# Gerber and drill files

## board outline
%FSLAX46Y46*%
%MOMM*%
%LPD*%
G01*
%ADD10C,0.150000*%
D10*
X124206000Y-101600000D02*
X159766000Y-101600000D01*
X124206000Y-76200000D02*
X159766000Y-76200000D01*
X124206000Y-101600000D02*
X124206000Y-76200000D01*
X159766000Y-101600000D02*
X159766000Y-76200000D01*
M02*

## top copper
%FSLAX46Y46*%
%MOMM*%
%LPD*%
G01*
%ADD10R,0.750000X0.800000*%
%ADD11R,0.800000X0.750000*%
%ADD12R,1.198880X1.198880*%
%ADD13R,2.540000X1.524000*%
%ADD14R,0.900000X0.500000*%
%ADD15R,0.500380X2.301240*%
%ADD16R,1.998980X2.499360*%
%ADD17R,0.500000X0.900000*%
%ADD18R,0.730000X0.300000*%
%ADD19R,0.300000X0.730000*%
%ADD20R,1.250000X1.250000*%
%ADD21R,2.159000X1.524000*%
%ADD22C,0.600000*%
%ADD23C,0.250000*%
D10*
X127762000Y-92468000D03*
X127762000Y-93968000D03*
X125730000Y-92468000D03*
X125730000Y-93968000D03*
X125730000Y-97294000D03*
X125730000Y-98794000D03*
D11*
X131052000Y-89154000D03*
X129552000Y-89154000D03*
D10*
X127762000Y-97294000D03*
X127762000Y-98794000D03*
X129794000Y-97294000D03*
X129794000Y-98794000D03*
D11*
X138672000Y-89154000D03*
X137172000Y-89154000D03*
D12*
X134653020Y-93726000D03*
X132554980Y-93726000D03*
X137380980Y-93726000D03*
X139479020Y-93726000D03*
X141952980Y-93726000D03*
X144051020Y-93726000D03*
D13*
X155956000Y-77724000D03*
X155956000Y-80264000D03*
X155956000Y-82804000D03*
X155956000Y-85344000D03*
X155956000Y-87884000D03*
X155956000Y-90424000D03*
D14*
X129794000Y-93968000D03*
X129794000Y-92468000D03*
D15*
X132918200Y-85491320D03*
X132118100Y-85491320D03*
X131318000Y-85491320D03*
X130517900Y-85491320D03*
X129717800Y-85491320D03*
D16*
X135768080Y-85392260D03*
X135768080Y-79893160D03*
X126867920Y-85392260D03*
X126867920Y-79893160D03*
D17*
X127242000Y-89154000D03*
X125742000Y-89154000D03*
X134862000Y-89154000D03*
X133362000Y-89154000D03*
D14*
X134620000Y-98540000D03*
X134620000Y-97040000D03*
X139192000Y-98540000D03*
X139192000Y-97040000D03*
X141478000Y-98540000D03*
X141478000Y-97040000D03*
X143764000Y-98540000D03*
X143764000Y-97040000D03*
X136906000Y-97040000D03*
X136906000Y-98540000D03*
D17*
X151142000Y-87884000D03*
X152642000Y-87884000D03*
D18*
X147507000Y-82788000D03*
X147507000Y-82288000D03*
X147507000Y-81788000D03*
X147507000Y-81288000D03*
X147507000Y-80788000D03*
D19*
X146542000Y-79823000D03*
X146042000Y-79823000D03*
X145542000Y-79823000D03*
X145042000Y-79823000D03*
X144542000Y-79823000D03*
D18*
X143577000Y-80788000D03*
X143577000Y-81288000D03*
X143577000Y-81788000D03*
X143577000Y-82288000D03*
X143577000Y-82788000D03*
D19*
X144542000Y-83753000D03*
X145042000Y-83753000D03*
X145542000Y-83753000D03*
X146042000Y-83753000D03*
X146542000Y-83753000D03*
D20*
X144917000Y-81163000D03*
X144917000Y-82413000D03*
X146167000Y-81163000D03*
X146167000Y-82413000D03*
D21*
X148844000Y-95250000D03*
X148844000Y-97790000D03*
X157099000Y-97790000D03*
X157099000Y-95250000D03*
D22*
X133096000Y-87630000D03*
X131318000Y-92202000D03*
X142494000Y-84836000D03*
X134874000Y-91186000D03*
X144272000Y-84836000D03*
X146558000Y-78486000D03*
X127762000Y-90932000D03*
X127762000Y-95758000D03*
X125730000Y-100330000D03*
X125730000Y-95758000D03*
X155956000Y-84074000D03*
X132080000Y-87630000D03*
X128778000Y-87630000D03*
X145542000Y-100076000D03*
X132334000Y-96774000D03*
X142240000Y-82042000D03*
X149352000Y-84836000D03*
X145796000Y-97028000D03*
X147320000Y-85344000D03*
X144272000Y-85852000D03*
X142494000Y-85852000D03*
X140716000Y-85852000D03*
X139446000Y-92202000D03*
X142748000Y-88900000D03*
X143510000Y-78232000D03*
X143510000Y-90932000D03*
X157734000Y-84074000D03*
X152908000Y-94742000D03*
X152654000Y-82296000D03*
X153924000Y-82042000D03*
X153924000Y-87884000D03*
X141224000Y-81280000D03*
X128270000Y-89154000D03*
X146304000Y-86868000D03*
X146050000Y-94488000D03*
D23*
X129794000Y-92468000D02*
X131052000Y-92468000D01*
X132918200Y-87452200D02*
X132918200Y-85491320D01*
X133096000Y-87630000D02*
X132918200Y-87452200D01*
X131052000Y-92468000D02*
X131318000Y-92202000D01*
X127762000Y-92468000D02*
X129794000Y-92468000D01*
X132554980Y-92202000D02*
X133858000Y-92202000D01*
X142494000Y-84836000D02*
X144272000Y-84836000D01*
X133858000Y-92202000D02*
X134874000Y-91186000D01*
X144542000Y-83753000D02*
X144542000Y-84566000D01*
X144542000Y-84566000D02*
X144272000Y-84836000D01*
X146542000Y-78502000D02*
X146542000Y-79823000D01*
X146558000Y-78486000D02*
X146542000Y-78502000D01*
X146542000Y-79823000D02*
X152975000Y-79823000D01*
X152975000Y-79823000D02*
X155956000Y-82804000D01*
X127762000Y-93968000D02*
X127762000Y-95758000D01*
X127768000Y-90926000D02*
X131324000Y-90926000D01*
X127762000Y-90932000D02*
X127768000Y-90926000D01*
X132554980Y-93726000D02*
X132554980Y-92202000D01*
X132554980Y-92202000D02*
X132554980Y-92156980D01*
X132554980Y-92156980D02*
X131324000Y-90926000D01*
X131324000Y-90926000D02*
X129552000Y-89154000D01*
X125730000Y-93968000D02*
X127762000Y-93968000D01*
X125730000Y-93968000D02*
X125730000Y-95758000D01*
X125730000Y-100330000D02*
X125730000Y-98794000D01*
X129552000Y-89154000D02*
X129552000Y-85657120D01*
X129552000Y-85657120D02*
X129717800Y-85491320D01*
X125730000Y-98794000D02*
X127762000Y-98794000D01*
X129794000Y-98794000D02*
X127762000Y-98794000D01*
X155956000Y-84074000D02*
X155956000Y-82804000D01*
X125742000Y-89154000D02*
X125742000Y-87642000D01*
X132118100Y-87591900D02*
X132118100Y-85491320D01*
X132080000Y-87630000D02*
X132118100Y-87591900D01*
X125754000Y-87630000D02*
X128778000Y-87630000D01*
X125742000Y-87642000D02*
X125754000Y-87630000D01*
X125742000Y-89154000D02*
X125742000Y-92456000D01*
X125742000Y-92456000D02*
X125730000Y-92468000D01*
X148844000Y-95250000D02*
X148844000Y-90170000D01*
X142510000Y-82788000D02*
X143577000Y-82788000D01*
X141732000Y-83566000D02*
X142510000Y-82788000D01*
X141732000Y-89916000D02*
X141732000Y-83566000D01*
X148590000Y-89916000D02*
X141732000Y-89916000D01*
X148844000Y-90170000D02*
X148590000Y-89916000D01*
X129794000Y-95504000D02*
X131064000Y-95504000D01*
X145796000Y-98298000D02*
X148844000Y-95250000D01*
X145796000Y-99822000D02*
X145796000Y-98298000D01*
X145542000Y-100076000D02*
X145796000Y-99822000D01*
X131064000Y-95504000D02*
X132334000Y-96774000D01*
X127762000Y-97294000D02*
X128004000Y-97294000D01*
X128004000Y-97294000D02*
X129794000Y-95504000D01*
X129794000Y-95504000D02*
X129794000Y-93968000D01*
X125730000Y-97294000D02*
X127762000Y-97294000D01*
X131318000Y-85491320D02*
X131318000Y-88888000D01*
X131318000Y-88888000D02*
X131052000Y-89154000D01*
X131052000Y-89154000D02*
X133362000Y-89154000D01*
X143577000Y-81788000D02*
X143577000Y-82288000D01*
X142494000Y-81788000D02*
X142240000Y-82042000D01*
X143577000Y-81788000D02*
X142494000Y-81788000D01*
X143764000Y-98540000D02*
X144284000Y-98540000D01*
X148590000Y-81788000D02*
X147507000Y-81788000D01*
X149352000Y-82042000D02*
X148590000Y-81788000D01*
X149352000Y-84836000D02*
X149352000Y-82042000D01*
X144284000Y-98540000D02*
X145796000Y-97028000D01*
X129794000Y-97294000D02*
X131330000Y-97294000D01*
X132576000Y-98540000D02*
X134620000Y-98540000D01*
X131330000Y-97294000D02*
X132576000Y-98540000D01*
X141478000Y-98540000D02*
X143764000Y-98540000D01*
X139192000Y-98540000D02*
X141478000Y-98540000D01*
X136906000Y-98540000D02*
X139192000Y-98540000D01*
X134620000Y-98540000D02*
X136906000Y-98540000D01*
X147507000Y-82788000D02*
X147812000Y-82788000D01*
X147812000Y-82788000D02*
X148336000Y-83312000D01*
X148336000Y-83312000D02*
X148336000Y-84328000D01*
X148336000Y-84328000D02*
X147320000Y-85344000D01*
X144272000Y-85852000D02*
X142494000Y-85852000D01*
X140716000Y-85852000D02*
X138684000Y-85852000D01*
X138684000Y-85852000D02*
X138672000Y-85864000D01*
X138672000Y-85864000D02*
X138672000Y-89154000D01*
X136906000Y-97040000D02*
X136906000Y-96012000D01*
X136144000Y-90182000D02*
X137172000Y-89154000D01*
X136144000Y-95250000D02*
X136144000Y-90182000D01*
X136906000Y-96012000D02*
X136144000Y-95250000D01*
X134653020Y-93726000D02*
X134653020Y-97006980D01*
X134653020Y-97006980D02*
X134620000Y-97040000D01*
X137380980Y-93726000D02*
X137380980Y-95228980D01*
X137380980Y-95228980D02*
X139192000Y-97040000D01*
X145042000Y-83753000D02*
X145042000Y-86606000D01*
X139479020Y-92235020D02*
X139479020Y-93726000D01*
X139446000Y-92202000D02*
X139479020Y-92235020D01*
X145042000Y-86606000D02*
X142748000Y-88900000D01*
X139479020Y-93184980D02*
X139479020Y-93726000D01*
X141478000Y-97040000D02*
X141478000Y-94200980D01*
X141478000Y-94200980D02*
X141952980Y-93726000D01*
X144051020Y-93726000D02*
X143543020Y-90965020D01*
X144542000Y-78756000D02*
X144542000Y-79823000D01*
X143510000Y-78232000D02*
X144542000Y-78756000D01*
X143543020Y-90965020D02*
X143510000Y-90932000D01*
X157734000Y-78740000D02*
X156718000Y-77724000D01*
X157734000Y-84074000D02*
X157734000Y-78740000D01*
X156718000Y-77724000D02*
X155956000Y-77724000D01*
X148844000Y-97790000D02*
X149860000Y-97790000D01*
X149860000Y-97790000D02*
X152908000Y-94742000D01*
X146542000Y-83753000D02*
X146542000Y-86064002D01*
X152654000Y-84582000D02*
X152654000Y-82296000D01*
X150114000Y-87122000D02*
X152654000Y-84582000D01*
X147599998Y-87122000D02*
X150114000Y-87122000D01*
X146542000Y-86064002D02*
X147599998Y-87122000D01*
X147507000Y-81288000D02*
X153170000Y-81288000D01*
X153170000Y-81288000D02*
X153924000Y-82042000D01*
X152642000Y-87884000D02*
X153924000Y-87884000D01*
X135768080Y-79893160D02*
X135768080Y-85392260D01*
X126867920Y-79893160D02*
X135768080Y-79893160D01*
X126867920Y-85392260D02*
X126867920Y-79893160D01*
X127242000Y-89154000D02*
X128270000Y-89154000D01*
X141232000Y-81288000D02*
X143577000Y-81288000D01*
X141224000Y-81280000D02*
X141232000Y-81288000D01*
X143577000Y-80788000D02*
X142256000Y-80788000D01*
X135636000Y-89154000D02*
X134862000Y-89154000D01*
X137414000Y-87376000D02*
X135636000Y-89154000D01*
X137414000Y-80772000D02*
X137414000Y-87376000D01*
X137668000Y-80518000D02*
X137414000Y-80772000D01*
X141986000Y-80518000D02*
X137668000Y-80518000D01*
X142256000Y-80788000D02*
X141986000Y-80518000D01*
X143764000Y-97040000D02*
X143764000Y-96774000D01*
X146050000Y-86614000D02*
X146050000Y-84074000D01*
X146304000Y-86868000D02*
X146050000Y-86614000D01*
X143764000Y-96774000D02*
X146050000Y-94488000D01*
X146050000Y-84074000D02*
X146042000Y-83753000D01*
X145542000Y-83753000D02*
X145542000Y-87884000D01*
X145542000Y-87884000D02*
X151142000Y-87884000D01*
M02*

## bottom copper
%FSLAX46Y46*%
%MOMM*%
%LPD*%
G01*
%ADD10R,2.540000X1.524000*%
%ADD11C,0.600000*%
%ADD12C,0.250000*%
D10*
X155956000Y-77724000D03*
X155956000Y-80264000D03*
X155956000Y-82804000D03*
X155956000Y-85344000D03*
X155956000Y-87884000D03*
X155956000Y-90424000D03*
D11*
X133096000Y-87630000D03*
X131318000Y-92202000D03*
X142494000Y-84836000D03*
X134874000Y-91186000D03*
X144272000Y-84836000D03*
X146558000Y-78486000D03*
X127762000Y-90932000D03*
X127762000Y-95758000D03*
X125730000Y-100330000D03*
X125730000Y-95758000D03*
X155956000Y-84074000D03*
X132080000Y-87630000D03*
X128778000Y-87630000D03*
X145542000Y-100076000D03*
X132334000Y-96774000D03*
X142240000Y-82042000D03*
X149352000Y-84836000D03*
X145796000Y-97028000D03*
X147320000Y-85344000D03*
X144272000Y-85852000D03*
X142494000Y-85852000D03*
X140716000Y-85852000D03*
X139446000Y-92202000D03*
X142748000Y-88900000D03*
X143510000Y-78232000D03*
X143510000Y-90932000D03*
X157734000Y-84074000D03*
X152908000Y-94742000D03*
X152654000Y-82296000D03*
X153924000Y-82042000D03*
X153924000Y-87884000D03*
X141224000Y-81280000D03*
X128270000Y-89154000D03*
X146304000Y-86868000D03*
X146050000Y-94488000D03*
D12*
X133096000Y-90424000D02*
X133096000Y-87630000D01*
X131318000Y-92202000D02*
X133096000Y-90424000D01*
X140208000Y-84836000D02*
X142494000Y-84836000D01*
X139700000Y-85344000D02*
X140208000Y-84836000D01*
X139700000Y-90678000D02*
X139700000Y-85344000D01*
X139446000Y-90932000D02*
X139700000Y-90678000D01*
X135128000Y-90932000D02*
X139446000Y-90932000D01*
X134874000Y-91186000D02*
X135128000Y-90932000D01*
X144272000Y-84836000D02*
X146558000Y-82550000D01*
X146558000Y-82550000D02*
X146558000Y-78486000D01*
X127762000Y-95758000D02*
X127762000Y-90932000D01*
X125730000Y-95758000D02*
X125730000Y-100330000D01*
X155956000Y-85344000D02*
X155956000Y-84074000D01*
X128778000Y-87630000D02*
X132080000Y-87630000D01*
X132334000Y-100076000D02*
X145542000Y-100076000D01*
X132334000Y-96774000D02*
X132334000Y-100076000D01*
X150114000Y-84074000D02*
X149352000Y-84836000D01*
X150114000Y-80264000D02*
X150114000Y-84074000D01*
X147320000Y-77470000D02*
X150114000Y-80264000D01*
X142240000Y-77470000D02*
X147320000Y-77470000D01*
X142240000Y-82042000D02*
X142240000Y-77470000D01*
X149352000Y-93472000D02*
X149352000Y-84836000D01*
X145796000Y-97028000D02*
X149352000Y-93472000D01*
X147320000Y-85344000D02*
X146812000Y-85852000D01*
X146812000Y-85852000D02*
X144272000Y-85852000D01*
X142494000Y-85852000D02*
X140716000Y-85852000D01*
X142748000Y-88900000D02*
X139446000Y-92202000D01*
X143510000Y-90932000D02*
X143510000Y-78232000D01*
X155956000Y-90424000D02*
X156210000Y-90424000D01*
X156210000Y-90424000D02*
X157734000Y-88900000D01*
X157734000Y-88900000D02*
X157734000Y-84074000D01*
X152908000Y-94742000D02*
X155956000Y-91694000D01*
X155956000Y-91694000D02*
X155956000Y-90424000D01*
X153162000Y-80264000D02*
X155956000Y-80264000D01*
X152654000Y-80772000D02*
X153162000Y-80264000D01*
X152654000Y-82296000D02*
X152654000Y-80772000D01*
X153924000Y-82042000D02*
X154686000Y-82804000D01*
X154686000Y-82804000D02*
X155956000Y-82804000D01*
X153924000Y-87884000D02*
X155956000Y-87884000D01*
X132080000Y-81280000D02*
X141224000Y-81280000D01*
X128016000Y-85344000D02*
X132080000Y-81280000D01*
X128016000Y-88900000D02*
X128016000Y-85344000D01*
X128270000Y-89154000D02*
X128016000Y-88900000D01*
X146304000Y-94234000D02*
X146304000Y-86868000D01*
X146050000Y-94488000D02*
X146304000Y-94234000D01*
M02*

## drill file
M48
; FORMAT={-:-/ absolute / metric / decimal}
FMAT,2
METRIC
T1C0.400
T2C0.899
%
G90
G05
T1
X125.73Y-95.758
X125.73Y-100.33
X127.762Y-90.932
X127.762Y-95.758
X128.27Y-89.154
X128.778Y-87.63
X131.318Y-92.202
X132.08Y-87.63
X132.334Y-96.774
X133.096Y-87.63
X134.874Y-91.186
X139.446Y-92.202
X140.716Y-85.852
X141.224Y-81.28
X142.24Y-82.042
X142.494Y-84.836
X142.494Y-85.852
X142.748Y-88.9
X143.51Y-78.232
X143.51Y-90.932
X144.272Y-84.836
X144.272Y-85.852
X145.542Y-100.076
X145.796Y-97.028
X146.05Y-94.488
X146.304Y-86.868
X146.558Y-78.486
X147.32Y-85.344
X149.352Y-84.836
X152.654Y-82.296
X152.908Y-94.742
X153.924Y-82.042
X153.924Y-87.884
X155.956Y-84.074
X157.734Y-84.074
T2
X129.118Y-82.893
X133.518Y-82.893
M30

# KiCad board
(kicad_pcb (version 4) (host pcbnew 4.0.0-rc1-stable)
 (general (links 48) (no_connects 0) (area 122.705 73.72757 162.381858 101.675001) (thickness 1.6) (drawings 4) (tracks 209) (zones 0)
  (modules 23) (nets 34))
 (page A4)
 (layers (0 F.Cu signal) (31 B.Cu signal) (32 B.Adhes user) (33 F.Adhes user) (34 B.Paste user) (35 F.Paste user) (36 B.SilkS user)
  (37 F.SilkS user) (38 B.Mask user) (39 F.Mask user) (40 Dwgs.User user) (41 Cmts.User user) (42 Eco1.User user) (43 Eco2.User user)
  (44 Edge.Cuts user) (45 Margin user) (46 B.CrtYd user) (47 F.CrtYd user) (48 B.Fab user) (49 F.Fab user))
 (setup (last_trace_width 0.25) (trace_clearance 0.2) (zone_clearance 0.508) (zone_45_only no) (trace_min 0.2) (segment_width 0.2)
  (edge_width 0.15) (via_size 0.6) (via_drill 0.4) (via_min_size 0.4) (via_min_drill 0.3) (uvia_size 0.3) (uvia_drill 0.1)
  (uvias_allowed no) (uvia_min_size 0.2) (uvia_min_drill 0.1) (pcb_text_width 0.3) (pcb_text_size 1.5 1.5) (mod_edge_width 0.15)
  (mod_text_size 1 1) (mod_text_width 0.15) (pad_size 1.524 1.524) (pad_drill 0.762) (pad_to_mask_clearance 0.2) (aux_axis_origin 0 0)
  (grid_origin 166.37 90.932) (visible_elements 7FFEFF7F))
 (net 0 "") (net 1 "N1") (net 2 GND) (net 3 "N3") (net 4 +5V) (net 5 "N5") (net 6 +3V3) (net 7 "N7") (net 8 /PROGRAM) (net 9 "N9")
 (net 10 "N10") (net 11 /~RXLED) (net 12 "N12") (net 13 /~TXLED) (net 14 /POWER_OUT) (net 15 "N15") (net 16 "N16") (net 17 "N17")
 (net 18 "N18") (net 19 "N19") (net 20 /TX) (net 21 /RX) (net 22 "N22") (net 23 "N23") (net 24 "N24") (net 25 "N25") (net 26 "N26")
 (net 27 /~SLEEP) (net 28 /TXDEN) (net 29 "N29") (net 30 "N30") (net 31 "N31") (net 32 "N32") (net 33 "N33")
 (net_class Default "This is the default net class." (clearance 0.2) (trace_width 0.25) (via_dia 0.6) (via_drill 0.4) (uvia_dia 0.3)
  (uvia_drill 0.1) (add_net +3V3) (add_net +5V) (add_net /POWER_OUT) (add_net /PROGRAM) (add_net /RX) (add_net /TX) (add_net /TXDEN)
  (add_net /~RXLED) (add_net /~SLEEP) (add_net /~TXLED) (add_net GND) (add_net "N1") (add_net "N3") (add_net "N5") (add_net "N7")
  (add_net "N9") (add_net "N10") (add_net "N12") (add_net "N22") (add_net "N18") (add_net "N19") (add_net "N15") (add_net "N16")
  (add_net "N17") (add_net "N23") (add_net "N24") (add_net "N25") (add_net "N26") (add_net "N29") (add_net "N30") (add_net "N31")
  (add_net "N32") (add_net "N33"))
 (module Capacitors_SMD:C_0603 (layer F.Cu) (at 127.762 93.218 270)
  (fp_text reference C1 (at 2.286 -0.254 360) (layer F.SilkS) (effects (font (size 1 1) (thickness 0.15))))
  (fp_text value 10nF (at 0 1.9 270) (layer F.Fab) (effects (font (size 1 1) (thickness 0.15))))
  (pad 1 smd rect (at -0.75 0 270) (size 0.8 0.75) (layers F.Cu F.Paste F.Mask) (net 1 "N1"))
  (pad 2 smd rect (at 0.75 0 270) (size 0.8 0.75) (layers F.Cu F.Paste F.Mask) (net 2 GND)))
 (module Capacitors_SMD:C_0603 (layer F.Cu) (at 125.73 93.218 270)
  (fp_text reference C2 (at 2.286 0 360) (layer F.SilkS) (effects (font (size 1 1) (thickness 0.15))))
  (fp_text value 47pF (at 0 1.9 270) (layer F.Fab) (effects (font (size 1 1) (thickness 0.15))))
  (pad 1 smd rect (at -0.75 0 270) (size 0.8 0.75) (layers F.Cu F.Paste F.Mask) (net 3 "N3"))
  (pad 2 smd rect (at 0.75 0 270) (size 0.8 0.75) (layers F.Cu F.Paste F.Mask) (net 2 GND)))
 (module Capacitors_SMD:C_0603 (layer F.Cu) (at 125.73 98.044 270)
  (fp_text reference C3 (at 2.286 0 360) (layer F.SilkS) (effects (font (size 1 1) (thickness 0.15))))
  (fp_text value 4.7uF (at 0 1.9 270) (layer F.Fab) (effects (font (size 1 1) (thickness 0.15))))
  (pad 1 smd rect (at -0.75 0 270) (size 0.8 0.75) (layers F.Cu F.Paste F.Mask) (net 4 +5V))
  (pad 2 smd rect (at 0.75 0 270) (size 0.8 0.75) (layers F.Cu F.Paste F.Mask) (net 2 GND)))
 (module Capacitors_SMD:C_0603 (layer F.Cu) (at 130.302 89.154 180)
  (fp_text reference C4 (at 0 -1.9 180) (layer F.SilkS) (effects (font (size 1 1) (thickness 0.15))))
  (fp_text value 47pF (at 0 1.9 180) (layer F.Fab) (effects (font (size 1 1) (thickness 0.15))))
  (pad 1 smd rect (at -0.75 0 180) (size 0.8 0.75) (layers F.Cu F.Paste F.Mask) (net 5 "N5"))
  (pad 2 smd rect (at 0.75 0 180) (size 0.8 0.75) (layers F.Cu F.Paste F.Mask) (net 2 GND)))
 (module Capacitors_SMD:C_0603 (layer F.Cu) (at 127.762 98.044 270)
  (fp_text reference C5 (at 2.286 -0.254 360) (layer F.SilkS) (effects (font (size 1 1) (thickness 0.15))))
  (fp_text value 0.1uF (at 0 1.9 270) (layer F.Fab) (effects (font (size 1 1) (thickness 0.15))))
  (pad 1 smd rect (at -0.75 0 270) (size 0.8 0.75) (layers F.Cu F.Paste F.Mask) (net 4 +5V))
  (pad 2 smd rect (at 0.75 0 270) (size 0.8 0.75) (layers F.Cu F.Paste F.Mask) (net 2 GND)))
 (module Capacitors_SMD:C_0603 (layer F.Cu) (at 129.794 98.044 270)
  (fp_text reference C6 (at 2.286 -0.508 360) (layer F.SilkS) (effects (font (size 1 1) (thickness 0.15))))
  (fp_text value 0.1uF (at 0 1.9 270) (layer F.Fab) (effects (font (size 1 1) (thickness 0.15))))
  (pad 1 smd rect (at -0.75 0 270) (size 0.8 0.75) (layers F.Cu F.Paste F.Mask) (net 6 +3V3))
  (pad 2 smd rect (at 0.75 0 270) (size 0.8 0.75) (layers F.Cu F.Paste F.Mask) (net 2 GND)))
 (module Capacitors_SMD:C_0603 (layer F.Cu) (at 137.922 89.154 180)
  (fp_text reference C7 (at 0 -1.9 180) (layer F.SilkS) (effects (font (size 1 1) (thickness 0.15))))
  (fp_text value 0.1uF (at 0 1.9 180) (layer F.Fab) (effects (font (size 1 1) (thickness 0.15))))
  (pad 1 smd rect (at -0.75 0 180) (size 0.8 0.75) (layers F.Cu F.Paste F.Mask) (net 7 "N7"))
  (pad 2 smd rect (at 0.75 0 180) (size 0.8 0.75) (layers F.Cu F.Paste F.Mask) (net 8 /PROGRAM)))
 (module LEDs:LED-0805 (layer F.Cu) (at 133.604 93.726)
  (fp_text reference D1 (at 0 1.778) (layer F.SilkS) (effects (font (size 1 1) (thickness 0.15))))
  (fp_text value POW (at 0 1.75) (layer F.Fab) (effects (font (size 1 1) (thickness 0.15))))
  (pad 2 smd rect (at 1.04902 0 180) (size 1.19888 1.19888) (layers F.Cu F.Paste F.Mask) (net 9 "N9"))
  (pad 1 smd rect (at -1.04902 0 180) (size 1.19888 1.19888) (layers F.Cu F.Paste F.Mask) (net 2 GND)))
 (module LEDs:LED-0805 (layer F.Cu) (at 138.43 93.726 180)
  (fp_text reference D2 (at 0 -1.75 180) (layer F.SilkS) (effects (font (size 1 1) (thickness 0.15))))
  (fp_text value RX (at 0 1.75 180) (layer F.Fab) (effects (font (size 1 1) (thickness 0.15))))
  (pad 2 smd rect (at 1.04902 0) (size 1.19888 1.19888) (layers F.Cu F.Paste F.Mask) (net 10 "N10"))
  (pad 1 smd rect (at -1.04902 0) (size 1.19888 1.19888) (layers F.Cu F.Paste F.Mask) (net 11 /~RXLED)))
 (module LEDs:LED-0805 (layer F.Cu) (at 143.002 93.726 180)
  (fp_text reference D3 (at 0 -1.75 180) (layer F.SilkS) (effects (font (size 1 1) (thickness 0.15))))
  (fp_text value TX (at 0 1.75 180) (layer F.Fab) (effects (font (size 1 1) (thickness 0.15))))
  (pad 2 smd rect (at 1.04902 0) (size 1.19888 1.19888) (layers F.Cu F.Paste F.Mask) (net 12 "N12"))
  (pad 1 smd rect (at -1.04902 0) (size 1.19888 1.19888) (layers F.Cu F.Paste F.Mask) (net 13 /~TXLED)))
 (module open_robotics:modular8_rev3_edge (layer F.Cu) (at 155.956 82.804 270)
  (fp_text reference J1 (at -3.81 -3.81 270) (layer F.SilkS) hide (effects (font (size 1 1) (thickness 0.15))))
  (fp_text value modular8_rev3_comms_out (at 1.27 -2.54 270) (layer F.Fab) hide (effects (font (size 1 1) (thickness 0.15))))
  (pad 1 smd rect (at -5.08 0 270) (size 1.524 2.54) (layers F.Cu F.Paste F.Mask) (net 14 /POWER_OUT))
  (pad 3 smd rect (at -2.54 0 270) (size 1.524 2.54) (layers F.Cu F.Paste F.Mask) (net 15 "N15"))
  (pad 5 smd rect (at 0 0 270) (size 1.524 2.54) (layers F.Cu F.Paste F.Mask) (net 2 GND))
  (pad 7 smd rect (at 2.54 0 270) (size 1.524 2.54) (layers F.Cu F.Paste F.Mask) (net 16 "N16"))
  (pad 9 smd rect (at 5.08 0 270) (size 1.524 2.54) (layers F.Cu F.Paste F.Mask) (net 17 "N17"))
  (pad 11 smd rect (at 7.62 0 270) (size 1.524 2.54) (layers F.Cu F.Paste F.Mask) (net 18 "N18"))
  (pad 2 smd rect (at -5.08 0 270) (size 1.524 2.54) (layers B.Cu F.Paste F.Mask) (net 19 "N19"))
  (pad 4 smd rect (at -2.54 0 270) (size 1.524 2.54) (layers B.Cu F.Paste F.Mask) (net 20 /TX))
  (pad 6 smd rect (at 0 0 270) (size 1.524 2.54) (layers B.Cu F.Paste F.Mask) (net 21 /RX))
  (pad 8 smd rect (at 2.54 0 270) (size 1.524 2.54) (layers B.Cu F.Paste F.Mask) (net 2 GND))
  (pad 10 smd rect (at 5.08 0 270) (size 1.524 2.54) (layers B.Cu F.Paste F.Mask) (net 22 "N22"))
  (pad 12 smd rect (at 7.62 0 270) (size 1.524 2.54) (layers B.Cu F.Paste F.Mask) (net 14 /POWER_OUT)))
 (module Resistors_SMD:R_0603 (layer F.Cu) (at 129.794 93.218 90)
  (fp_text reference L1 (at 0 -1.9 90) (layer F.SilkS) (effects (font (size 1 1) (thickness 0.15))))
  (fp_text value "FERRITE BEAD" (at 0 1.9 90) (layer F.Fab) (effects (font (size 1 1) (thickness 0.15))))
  (pad 1 smd rect (at -0.75 0 90) (size 0.5 0.9) (layers F.Cu F.Paste F.Mask) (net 4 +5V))
  (pad 2 smd rect (at 0.75 0 90) (size 0.5 0.9) (layers F.Cu F.Paste F.Mask) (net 1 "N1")))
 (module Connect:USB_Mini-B (layer F.Cu) (at 131.318 82.042 270)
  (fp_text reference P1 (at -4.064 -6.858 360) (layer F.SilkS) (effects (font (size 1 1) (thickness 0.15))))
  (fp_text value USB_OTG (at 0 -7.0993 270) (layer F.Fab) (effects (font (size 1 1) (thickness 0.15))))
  (pad 1 smd rect (at 3.44932 -1.6002 270) (size 2.30124 0.50038) (layers F.Cu F.Paste F.Mask) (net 1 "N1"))
  (pad 2 smd rect (at 3.44932 -0.8001 270) (size 2.30124 0.50038) (layers F.Cu F.Paste F.Mask) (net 3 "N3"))
  (pad 3 smd rect (at 3.44932 0 270) (size 2.30124 0.50038) (layers F.Cu F.Paste F.Mask) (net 5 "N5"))
  (pad 4 smd rect (at 3.44932 0.8001 270) (size 2.30124 0.50038) (layers F.Cu F.Paste F.Mask) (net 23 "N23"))
  (pad 5 smd rect (at 3.44932 1.6002 270) (size 2.30124 0.50038) (layers F.Cu F.Paste F.Mask) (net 2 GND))
  (pad 6 smd rect (at 3.35026 -4.45008 270) (size 2.49936 1.99898) (layers F.Cu F.Paste F.Mask) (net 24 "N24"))
  (pad 6 smd rect (at -2.14884 -4.45008 270) (size 2.49936 1.99898) (layers F.Cu F.Paste F.Mask) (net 24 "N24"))
  (pad 6 smd rect (at 3.35026 4.45008 270) (size 2.49936 1.99898) (layers F.Cu F.Paste F.Mask) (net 24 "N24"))
  (pad 6 smd rect (at -2.14884 4.45008 270) (size 2.49936 1.99898) (layers F.Cu F.Paste F.Mask) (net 24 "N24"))
  (pad "" np_thru_hole circle (at 0.8509 -2.19964 270) (size 0.89916 0.89916) (drill 0.89916) (layers *.Cu *.Mask F.SilkS))
  (pad "" np_thru_hole circle (at 0.8509 2.19964 270) (size 0.89916 0.89916) (drill 0.89916) (layers *.Cu *.Mask F.SilkS)))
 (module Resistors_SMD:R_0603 (layer F.Cu) (at 126.492 89.154 180)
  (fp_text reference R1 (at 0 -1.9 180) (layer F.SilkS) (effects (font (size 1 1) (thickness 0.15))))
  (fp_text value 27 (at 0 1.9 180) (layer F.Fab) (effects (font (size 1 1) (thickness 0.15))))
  (pad 1 smd rect (at -0.75 0 180) (size 0.5 0.9) (layers F.Cu F.Paste F.Mask) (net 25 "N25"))
  (pad 2 smd rect (at 0.75 0 180) (size 0.5 0.9) (layers F.Cu F.Paste F.Mask) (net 3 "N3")))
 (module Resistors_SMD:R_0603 (layer F.Cu) (at 134.112 89.154 180)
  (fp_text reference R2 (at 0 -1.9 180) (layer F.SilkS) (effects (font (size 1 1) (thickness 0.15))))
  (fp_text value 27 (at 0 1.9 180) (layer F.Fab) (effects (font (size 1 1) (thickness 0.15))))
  (pad 1 smd rect (at -0.75 0 180) (size 0.5 0.9) (layers F.Cu F.Paste F.Mask) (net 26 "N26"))
  (pad 2 smd rect (at 0.75 0 180) (size 0.5 0.9) (layers F.Cu F.Paste F.Mask) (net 5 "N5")))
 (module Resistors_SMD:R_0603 (layer F.Cu) (at 134.62 97.79 90)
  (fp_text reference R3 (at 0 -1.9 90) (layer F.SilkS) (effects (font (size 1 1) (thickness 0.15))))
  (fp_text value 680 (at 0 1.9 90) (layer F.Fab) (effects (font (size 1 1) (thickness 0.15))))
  (pad 1 smd rect (at -0.75 0 90) (size 0.5 0.9) (layers F.Cu F.Paste F.Mask) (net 6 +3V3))
  (pad 2 smd rect (at 0.75 0 90) (size 0.5 0.9) (layers F.Cu F.Paste F.Mask) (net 9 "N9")))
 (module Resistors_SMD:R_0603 (layer F.Cu) (at 139.192 97.79 90)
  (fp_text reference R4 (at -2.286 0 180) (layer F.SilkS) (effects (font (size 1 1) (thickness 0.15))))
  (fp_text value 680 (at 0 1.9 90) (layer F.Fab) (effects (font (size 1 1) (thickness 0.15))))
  (pad 1 smd rect (at -0.75 0 90) (size 0.5 0.9) (layers F.Cu F.Paste F.Mask) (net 6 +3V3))
  (pad 2 smd rect (at 0.75 0 90) (size 0.5 0.9) (layers F.Cu F.Paste F.Mask) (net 10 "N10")))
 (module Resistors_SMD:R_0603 (layer F.Cu) (at 141.478 97.79 90)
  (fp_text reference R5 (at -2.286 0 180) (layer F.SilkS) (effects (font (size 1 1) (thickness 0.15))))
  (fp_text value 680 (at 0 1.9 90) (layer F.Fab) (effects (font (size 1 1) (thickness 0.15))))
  (pad 1 smd rect (at -0.75 0 90) (size 0.5 0.9) (layers F.Cu F.Paste F.Mask) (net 6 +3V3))
  (pad 2 smd rect (at 0.75 0 90) (size 0.5 0.9) (layers F.Cu F.Paste F.Mask) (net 12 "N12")))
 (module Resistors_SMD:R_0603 (layer F.Cu) (at 143.764 97.79 90)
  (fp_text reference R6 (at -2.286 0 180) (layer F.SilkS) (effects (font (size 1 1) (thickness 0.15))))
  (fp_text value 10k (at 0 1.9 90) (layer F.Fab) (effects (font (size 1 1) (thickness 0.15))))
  (pad 1 smd rect (at -0.75 0 90) (size 0.5 0.9) (layers F.Cu F.Paste F.Mask) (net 6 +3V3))
  (pad 2 smd rect (at 0.75 0 90) (size 0.5 0.9) (layers F.Cu F.Paste F.Mask) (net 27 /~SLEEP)))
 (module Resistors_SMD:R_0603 (layer F.Cu) (at 136.906 97.79 270)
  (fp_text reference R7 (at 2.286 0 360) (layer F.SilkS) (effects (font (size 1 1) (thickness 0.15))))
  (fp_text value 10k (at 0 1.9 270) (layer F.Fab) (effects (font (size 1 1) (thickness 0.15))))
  (pad 1 smd rect (at -0.75 0 270) (size 0.5 0.9) (layers F.Cu F.Paste F.Mask) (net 8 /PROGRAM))
  (pad 2 smd rect (at 0.75 0 270) (size 0.5 0.9) (layers F.Cu F.Paste F.Mask) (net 6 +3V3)))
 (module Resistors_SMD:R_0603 (layer F.Cu) (at 151.892 87.884)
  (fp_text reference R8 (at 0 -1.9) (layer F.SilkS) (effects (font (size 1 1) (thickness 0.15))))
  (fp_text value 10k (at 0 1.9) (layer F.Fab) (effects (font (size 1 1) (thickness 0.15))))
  (pad 1 smd rect (at -0.75 0) (size 0.5 0.9) (layers F.Cu F.Paste F.Mask) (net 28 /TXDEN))
  (pad 2 smd rect (at 0.75 0) (size 0.5 0.9) (layers F.Cu F.Paste F.Mask) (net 22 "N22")))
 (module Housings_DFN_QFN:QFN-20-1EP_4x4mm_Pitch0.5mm (layer F.Cu) (at 145.542 81.788 180)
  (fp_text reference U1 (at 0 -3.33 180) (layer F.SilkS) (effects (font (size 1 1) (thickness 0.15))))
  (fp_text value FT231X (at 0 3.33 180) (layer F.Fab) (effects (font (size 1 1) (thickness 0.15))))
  (pad 1 smd rect (at -1.965 -1 180) (size 0.73 0.3) (layers F.Cu F.Paste F.Mask) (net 7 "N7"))
  (pad 2 smd rect (at -1.965 -0.5 180) (size 0.73 0.3) (layers F.Cu F.Paste F.Mask) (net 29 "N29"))
  (pad 3 smd rect (at -1.965 0 180) (size 0.73 0.3) (layers F.Cu F.Paste F.Mask) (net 6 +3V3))
  (pad 4 smd rect (at -1.965 0.5 180) (size 0.73 0.3) (layers F.Cu F.Paste F.Mask) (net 21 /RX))
  (pad 5 smd rect (at -1.965 1 180) (size 0.73 0.3) (layers F.Cu F.Paste F.Mask) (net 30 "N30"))
  (pad 6 smd rect (at -1 1.965 270) (size 0.73 0.3) (layers F.Cu F.Paste F.Mask) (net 2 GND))
  (pad 7 smd rect (at -0.5 1.965 270) (size 0.73 0.3) (layers F.Cu F.Paste F.Mask) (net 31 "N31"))
  (pad 8 smd rect (at 0 1.965 270) (size 0.73 0.3) (layers F.Cu F.Paste F.Mask) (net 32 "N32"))
  (pad 9 smd rect (at 0.5 1.965 270) (size 0.73 0.3) (layers F.Cu F.Paste F.Mask) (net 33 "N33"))
  (pad 10 smd rect (at 1 1.965 270) (size 0.73 0.3) (layers F.Cu F.Paste F.Mask) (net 13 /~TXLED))
  (pad 11 smd rect (at 1.965 1 180) (size 0.73 0.3) (layers F.Cu F.Paste F.Mask) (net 26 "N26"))
  (pad 12 smd rect (at 1.965 0.5 180) (size 0.73 0.3) (layers F.Cu F.Paste F.Mask) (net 25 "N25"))
  (pad 13 smd rect (at 1.965 0 180) (size 0.73 0.3) (layers F.Cu F.Paste F.Mask) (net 6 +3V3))
  (pad 14 smd rect (at 1.965 -0.5 180) (size 0.73 0.3) (layers F.Cu F.Paste F.Mask) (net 6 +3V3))
  (pad 15 smd rect (at 1.965 -1 180) (size 0.73 0.3) (layers F.Cu F.Paste F.Mask) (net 4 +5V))
  (pad 16 smd rect (at 1 -1.965 270) (size 0.73 0.3) (layers F.Cu F.Paste F.Mask) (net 2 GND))
  (pad 17 smd rect (at 0.5 -1.965 270) (size 0.73 0.3) (layers F.Cu F.Paste F.Mask) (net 11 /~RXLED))
  (pad 18 smd rect (at 0 -1.965 270) (size 0.73 0.3) (layers F.Cu F.Paste F.Mask) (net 28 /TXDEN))
  (pad 19 smd rect (at -0.5 -1.965 270) (size 0.73 0.3) (layers F.Cu F.Paste F.Mask) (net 27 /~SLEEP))
  (pad 20 smd rect (at -1 -1.965 270) (size 0.73 0.3) (layers F.Cu F.Paste F.Mask) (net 20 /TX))
  (pad 21 smd rect (at 0.625 0.625 180) (size 1.25 1.25) (layers F.Cu F.Paste F.Mask) (solder_paste_margin_ratio -0.2))
  (pad 21 smd rect (at 0.625 -0.625 180) (size 1.25 1.25) (layers F.Cu F.Paste F.Mask) (solder_paste_margin_ratio -0.2))
  (pad 21 smd rect (at -0.625 0.625 180) (size 1.25 1.25) (layers F.Cu F.Paste F.Mask) (solder_paste_margin_ratio -0.2))
  (pad 21 smd rect (at -0.625 -0.625 180) (size 1.25 1.25) (layers F.Cu F.Paste F.Mask) (solder_paste_margin_ratio -0.2)))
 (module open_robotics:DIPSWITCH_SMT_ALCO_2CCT (layer F.Cu) (at 148.844 95.25)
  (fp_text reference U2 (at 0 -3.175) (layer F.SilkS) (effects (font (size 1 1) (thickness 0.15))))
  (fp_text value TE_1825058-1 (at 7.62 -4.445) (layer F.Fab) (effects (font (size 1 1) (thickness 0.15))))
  (pad 1 smd rect (at 0 0) (size 2.159 1.524) (layers F.Cu F.Paste F.Mask) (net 4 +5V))
  (pad 2 smd rect (at 0 2.54) (size 2.159 1.524) (layers F.Cu F.Paste F.Mask) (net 14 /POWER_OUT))
  (pad 3 smd rect (at 8.255 2.54) (size 2.159 1.524) (layers F.Cu F.Paste F.Mask))
  (pad 4 smd rect (at 8.255 0) (size 2.159 1.524) (layers F.Cu F.Paste F.Mask)))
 (gr_line (start 124.206 101.6) (end 159.766 101.6) (angle 90) (layer Edge.Cuts) (width 0.15))
 (gr_line (start 124.206 76.2) (end 159.766 76.2) (angle 90) (layer Edge.Cuts) (width 0.15))
 (gr_line (start 124.206 101.6) (end 124.206 76.2) (angle 90) (layer Edge.Cuts) (width 0.15))
 (gr_line (start 159.766 101.6) (end 159.766 76.2) (angle 90) (layer Edge.Cuts) (width 0.15))
 (segment (start 129.794 92.468) (end 131.052 92.468) (width 0.25) (layer F.Cu) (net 1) (status 10))
 (segment (start 132.9182 87.4522) (end 132.9182 85.49132) (width 0.25) (layer F.Cu) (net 1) (status 20))
 (segment (start 133.096 87.63) (end 132.9182 87.4522) (width 0.25) (layer F.Cu) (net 1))
 (via (at 133.096 87.63) (size 0.6) (drill 0.4) (layers F.Cu B.Cu) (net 1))
 (segment (start 133.096 90.424) (end 133.096 87.63) (width 0.25) (layer B.Cu) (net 1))
 (segment (start 131.318 92.202) (end 133.096 90.424) (width 0.25) (layer B.Cu) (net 1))
 (via (at 131.318 92.202) (size 0.6) (drill 0.4) (layers F.Cu B.Cu) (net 1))
 (segment (start 131.052 92.468) (end 131.318 92.202) (width 0.25) (layer F.Cu) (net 1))
 (segment (start 127.762 92.468) (end 129.794 92.468) (width 0.25) (layer F.Cu) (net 1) (status 30))
 (segment (start 132.55498 92.202) (end 133.858 92.202) (width 0.25) (layer F.Cu) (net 2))
 (segment (start 142.494 84.836) (end 144.272 84.836) (width 0.25) (layer F.Cu) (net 2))
 (via (at 142.494 84.836) (size 0.6) (drill 0.4) (layers F.Cu B.Cu) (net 2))
 (segment (start 140.208 84.836) (end 142.494 84.836) (width 0.25) (layer B.Cu) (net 2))
 (segment (start 139.7 85.344) (end 140.208 84.836) (width 0.25) (layer B.Cu) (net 2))
 (segment (start 139.7 90.678) (end 139.7 85.344) (width 0.25) (layer B.Cu) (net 2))
 (segment (start 139.446 90.932) (end 139.7 90.678) (width 0.25) (layer B.Cu) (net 2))
 (segment (start 135.128 90.932) (end 139.446 90.932) (width 0.25) (layer B.Cu) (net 2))
 (segment (start 134.874 91.186) (end 135.128 90.932) (width 0.25) (layer B.Cu) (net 2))
 (via (at 134.874 91.186) (size 0.6) (drill 0.4) (layers F.Cu B.Cu) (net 2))
 (segment (start 133.858 92.202) (end 134.874 91.186) (width 0.25) (layer F.Cu) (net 2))
 (segment (start 144.542 83.753) (end 144.542 84.566) (width 0.25) (layer F.Cu) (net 2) (status 10))
 (segment (start 144.542 84.566) (end 144.272 84.836) (width 0.25) (layer F.Cu) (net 2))
 (segment (start 146.542 78.502) (end 146.542 79.823) (width 0.25) (layer F.Cu) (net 2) (status 20))
 (via (at 144.272 84.836) (size 0.6) (drill 0.4) (layers F.Cu B.Cu) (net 2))
 (segment (start 144.272 84.836) (end 146.558 82.55) (width 0.25) (layer B.Cu) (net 2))
 (segment (start 146.558 82.55) (end 146.558 78.486) (width 0.25) (layer B.Cu) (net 2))
 (via (at 146.558 78.486) (size 0.6) (drill 0.4) (layers F.Cu B.Cu) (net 2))
 (segment (start 146.558 78.486) (end 146.542 78.502) (width 0.25) (layer F.Cu) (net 2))
 (segment (start 146.542 79.823) (end 152.975 79.823) (width 0.25) (layer F.Cu) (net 2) (status 10))
 (segment (start 152.975 79.823) (end 155.956 82.804) (width 0.25) (layer F.Cu) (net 2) (status 20))
 (segment (start 127.762 93.968) (end 127.762 95.758) (width 0.25) (layer F.Cu) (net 2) (status 10))
 (segment (start 127.768 90.926) (end 131.324 90.926) (width 0.25) (layer F.Cu) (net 2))
 (segment (start 127.762 90.932) (end 127.768 90.926) (width 0.25) (layer F.Cu) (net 2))
 (via (at 127.762 90.932) (size 0.6) (drill 0.4) (layers F.Cu B.Cu) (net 2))
 (segment (start 127.762 95.758) (end 127.762 90.932) (width 0.25) (layer B.Cu) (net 2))
 (via (at 127.762 95.758) (size 0.6) (drill 0.4) (layers F.Cu B.Cu) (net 2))
 (segment (start 132.55498 93.726) (end 132.55498 92.202) (width 0.25) (layer F.Cu) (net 2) (status 10))
 (segment (start 132.55498 92.202) (end 132.55498 92.15698) (width 0.25) (layer F.Cu) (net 2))
 (segment (start 132.55498 92.15698) (end 131.324 90.926) (width 0.25) (layer F.Cu) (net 2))
 (segment (start 131.324 90.926) (end 129.552 89.154) (width 0.25) (layer F.Cu) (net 2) (status 20))
 (segment (start 125.73 93.968) (end 127.762 93.968) (width 0.25) (layer F.Cu) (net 2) (status 30))
 (segment (start 125.73 93.968) (end 125.73 95.758) (width 0.25) (layer F.Cu) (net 2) (status 10))
 (segment (start 125.73 100.33) (end 125.73 98.794) (width 0.25) (layer F.Cu) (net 2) (status 20))
 (via (at 125.73 100.33) (size 0.6) (drill 0.4) (layers F.Cu B.Cu) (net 2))
 (segment (start 125.73 95.758) (end 125.73 100.33) (width 0.25) (layer B.Cu) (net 2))
 (via (at 125.73 95.758) (size 0.6) (drill 0.4) (layers F.Cu B.Cu) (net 2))
 (segment (start 129.552 89.154) (end 129.552 85.65712) (width 0.25) (layer F.Cu) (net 2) (status 30))
 (segment (start 129.552 85.65712) (end 129.7178 85.49132) (width 0.25) (layer F.Cu) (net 2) (status 30))
 (segment (start 125.73 98.794) (end 127.762 98.794) (width 0.25) (layer F.Cu) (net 2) (status 30))
 (segment (start 129.794 98.794) (end 127.762 98.794) (width 0.25) (layer F.Cu) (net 2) (status 30))
 (segment (start 155.956 85.344) (end 155.956 84.074) (width 0.25) (layer B.Cu) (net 2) (status 10))
 (segment (start 155.956 84.074) (end 155.956 82.804) (width 0.25) (layer F.Cu) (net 2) (status 20))
 (via (at 155.956 84.074) (size 0.6) (drill 0.4) (layers F.Cu B.Cu) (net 2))
 (segment (start 125.742 89.154) (end 125.742 87.642) (width 0.25) (layer F.Cu) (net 3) (status 10))
 (segment (start 132.1181 87.5919) (end 132.1181 85.49132) (width 0.25) (layer F.Cu) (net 3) (status 20))
 (segment (start 132.08 87.63) (end 132.1181 87.5919) (width 0.25) (layer F.Cu) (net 3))
 (via (at 132.08 87.63) (size 0.6) (drill 0.4) (layers F.Cu B.Cu) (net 3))
 (segment (start 128.778 87.63) (end 132.08 87.63) (width 0.25) (layer B.Cu) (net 3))
 (via (at 128.778 87.63) (size 0.6) (drill 0.4) (layers F.Cu B.Cu) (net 3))
 (segment (start 125.754 87.63) (end 128.778 87.63) (width 0.25) (layer F.Cu) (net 3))
 (segment (start 125.742 87.642) (end 125.754 87.63) (width 0.25) (layer F.Cu) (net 3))
 (segment (start 125.742 89.154) (end 125.742 92.456) (width 0.25) (layer F.Cu) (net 3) (status 30))
 (segment (start 125.742 92.456) (end 125.73 92.468) (width 0.25) (layer F.Cu) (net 3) (status 30))
 (segment (start 148.844 95.25) (end 148.844 90.17) (width 0.25) (layer F.Cu) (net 4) (status 10))
 (segment (start 142.51 82.788) (end 143.577 82.788) (width 0.25) (layer F.Cu) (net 4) (status 20))
 (segment (start 141.732 83.566) (end 142.51 82.788) (width 0.25) (layer F.Cu) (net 4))
 (segment (start 141.732 89.916) (end 141.732 83.566) (width 0.25) (layer F.Cu) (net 4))
 (segment (start 148.59 89.916) (end 141.732 89.916) (width 0.25) (layer F.Cu) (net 4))
 (segment (start 148.844 90.17) (end 148.59 89.916) (width 0.25) (layer F.Cu) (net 4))
 (segment (start 129.794 95.504) (end 131.064 95.504) (width 0.25) (layer F.Cu) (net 4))
 (segment (start 145.796 98.298) (end 148.844 95.25) (width 0.25) (layer F.Cu) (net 4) (status 20))
 (segment (start 145.796 99.822) (end 145.796 98.298) (width 0.25) (layer F.Cu) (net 4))
 (segment (start 145.542 100.076) (end 145.796 99.822) (width 0.25) (layer F.Cu) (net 4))
 (via (at 145.542 100.076) (size 0.6) (drill 0.4) (layers F.Cu B.Cu) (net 4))
 (segment (start 132.334 100.076) (end 145.542 100.076) (width 0.25) (layer B.Cu) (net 4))
 (segment (start 132.334 96.774) (end 132.334 100.076) (width 0.25) (layer B.Cu) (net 4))
 (via (at 132.334 96.774) (size 0.6) (drill 0.4) (layers F.Cu B.Cu) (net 4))
 (segment (start 131.064 95.504) (end 132.334 96.774) (width 0.25) (layer F.Cu) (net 4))
 (segment (start 127.762 97.294) (end 128.004 97.294) (width 0.25) (layer F.Cu) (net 4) (status 30))
 (segment (start 128.004 97.294) (end 129.794 95.504) (width 0.25) (layer F.Cu) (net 4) (status 10))
 (segment (start 129.794 95.504) (end 129.794 93.968) (width 0.25) (layer F.Cu) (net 4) (status 20))
 (segment (start 125.73 97.294) (end 127.762 97.294) (width 0.25) (layer F.Cu) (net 4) (status 30))
 (segment (start 131.318 85.49132) (end 131.318 88.888) (width 0.25) (layer F.Cu) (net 5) (status 30))
 (segment (start 131.318 88.888) (end 131.052 89.154) (width 0.25) (layer F.Cu) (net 5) (status 30))
 (segment (start 131.052 89.154) (end 133.362 89.154) (width 0.25) (layer F.Cu) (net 5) (status 30))
 (segment (start 143.577 81.788) (end 143.577 82.288) (width 0.25) (layer F.Cu) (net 6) (status 30))
 (segment (start 150.114 84.074) (end 149.352 84.836) (width 0.25) (layer B.Cu) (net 6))
 (segment (start 150.114 80.264) (end 150.114 84.074) (width 0.25) (layer B.Cu) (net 6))
 (segment (start 147.32 77.47) (end 150.114 80.264) (width 0.25) (layer B.Cu) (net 6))
 (segment (start 142.24 77.47) (end 147.32 77.47) (width 0.25) (layer B.Cu) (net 6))
 (segment (start 142.24 82.042) (end 142.24 77.47) (width 0.25) (layer B.Cu) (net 6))
 (via (at 142.24 82.042) (size 0.6) (drill 0.4) (layers F.Cu B.Cu) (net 6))
 (segment (start 142.494 81.788) (end 142.24 82.042) (width 0.25) (layer F.Cu) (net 6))
 (segment (start 143.577 81.788) (end 142.494 81.788) (width 0.25) (layer F.Cu) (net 6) (status 10))
 (segment (start 143.764 98.54) (end 144.284 98.54) (width 0.25) (layer F.Cu) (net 6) (status 10))
 (segment (start 148.59 81.788) (end 147.507 81.788) (width 0.25) (layer F.Cu) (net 6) (status 20))
 (segment (start 149.352 82.042) (end 148.59 81.788) (width 0.25) (layer F.Cu) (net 6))
 (segment (start 149.352 84.836) (end 149.352 82.042) (width 0.25) (layer F.Cu) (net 6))
 (via (at 149.352 84.836) (size 0.6) (drill 0.4) (layers F.Cu B.Cu) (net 6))
 (segment (start 149.352 93.472) (end 149.352 84.836) (width 0.25) (layer B.Cu) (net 6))
 (segment (start 145.796 97.028) (end 149.352 93.472) (width 0.25) (layer B.Cu) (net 6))
 (via (at 145.796 97.028) (size 0.6) (drill 0.4) (layers F.Cu B.Cu) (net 6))
 (segment (start 144.284 98.54) (end 145.796 97.028) (width 0.25) (layer F.Cu) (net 6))
 (segment (start 129.794 97.294) (end 131.33 97.294) (width 0.25) (layer F.Cu) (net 6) (status 10))
 (segment (start 132.576 98.54) (end 134.62 98.54) (width 0.25) (layer F.Cu) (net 6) (status 20))
 (segment (start 131.33 97.294) (end 132.576 98.54) (width 0.25) (layer F.Cu) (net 6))
 (segment (start 141.478 98.54) (end 143.764 98.54) (width 0.25) (layer F.Cu) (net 6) (status 30))
 (segment (start 139.192 98.54) (end 141.478 98.54) (width 0.25) (layer F.Cu) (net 6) (status 30))
 (segment (start 136.906 98.54) (end 139.192 98.54) (width 0.25) (layer F.Cu) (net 6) (status 30))
 (segment (start 134.62 98.54) (end 136.906 98.54) (width 0.25) (layer F.Cu) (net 6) (status 30))
 (segment (start 147.507 82.788) (end 147.812 82.788) (width 0.25) (layer F.Cu) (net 7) (status 30))
 (segment (start 147.812 82.788) (end 148.336 83.312) (width 0.25) (layer F.Cu) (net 7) (status 10))
 (segment (start 148.336 83.312) (end 148.336 84.328) (width 0.25) (layer F.Cu) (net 7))
 (segment (start 148.336 84.328) (end 147.32 85.344) (width 0.25) (layer F.Cu) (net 7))
 (via (at 147.32 85.344) (size 0.6) (drill 0.4) (layers F.Cu B.Cu) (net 7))
 (segment (start 147.32 85.344) (end 146.812 85.852) (width 0.25) (layer B.Cu) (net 7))
 (segment (start 146.812 85.852) (end 144.272 85.852) (width 0.25) (layer B.Cu) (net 7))
 (via (at 144.272 85.852) (size 0.6) (drill 0.4) (layers F.Cu B.Cu) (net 7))
 (segment (start 144.272 85.852) (end 142.494 85.852) (width 0.25) (layer F.Cu) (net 7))
 (via (at 142.494 85.852) (size 0.6) (drill 0.4) (layers F.Cu B.Cu) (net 7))
 (segment (start 142.494 85.852) (end 140.716 85.852) (width 0.25) (layer B.Cu) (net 7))
 (via (at 140.716 85.852) (size 0.6) (drill 0.4) (layers F.Cu B.Cu) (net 7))
 (segment (start 140.716 85.852) (end 138.684 85.852) (width 0.25) (layer F.Cu) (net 7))
 (segment (start 138.684 85.852) (end 138.672 85.864) (width 0.25) (layer F.Cu) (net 7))
 (segment (start 138.672 85.864) (end 138.672 89.154) (width 0.25) (layer F.Cu) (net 7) (status 20))
 (segment (start 136.906 97.04) (end 136.906 96.012) (width 0.25) (layer F.Cu) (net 8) (status 10))
 (segment (start 136.144 90.182) (end 137.172 89.154) (width 0.25) (layer F.Cu) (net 8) (status 20))
 (segment (start 136.144 95.25) (end 136.144 90.182) (width 0.25) (layer F.Cu) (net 8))
 (segment (start 136.906 96.012) (end 136.144 95.25) (width 0.25) (layer F.Cu) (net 8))
 (segment (start 134.65302 93.726) (end 134.65302 97.00698) (width 0.25) (layer F.Cu) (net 9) (status 30))
 (segment (start 134.65302 97.00698) (end 134.62 97.04) (width 0.25) (layer F.Cu) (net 9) (status 30))
 (segment (start 137.38098 93.726) (end 137.38098 95.22898) (width 0.25) (layer F.Cu) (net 10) (status 10))
 (segment (start 137.38098 95.22898) (end 139.192 97.04) (width 0.25) (layer F.Cu) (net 10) (status 20))
 (segment (start 145.042 83.753) (end 145.042 86.606) (width 0.25) (layer F.Cu) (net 11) (status 400000))
 (segment (start 139.47902 92.23502) (end 139.47902 93.726) (width 0.25) (layer F.Cu) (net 11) (status 800000))
 (segment (start 139.446 92.202) (end 139.47902 92.23502) (width 0.25) (layer F.Cu) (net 11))
 (via (at 139.446 92.202) (size 0.6) (drill 0.4) (layers F.Cu B.Cu) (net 11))
 (segment (start 142.748 88.9) (end 139.446 92.202) (width 0.25) (layer B.Cu) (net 11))
 (via (at 142.748 88.9) (size 0.6) (drill 0.4) (layers F.Cu B.Cu) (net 11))
 (segment (start 145.042 86.606) (end 142.748 88.9) (width 0.25) (layer F.Cu) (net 11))
 (segment (start 139.47902 93.18498) (end 139.47902 93.726) (width 0.25) (layer F.Cu) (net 11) (status 30))
 (segment (start 141.478 97.04) (end 141.478 94.20098) (width 0.25) (layer F.Cu) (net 12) (status 30))
 (segment (start 141.478 94.20098) (end 141.95298 93.726) (width 0.25) (layer F.Cu) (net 12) (status 30))
 (segment (start 144.05102 93.726) (end 143.54302 90.96502) (width 0.25) (layer F.Cu) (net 13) (status 10))
 (segment (start 144.542 78.756) (end 144.542 79.823) (width 0.25) (layer F.Cu) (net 13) (status 20))
 (segment (start 143.51 78.232) (end 144.542 78.756) (width 0.25) (layer F.Cu) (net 13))
 (via (at 143.51 78.232) (size 0.6) (drill 0.4) (layers F.Cu B.Cu) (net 13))
 (segment (start 143.51 90.932) (end 143.51 78.232) (width 0.25) (layer B.Cu) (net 13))
 (via (at 143.51 90.932) (size 0.6) (drill 0.4) (layers F.Cu B.Cu) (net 13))
 (segment (start 143.54302 90.96502) (end 143.51 90.932) (width 0.25) (layer F.Cu) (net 13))
 (segment (start 155.956 90.424) (end 156.21 90.424) (width 0.25) (layer B.Cu) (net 14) (status 30))
 (segment (start 156.21 90.424) (end 157.734 88.9) (width 0.25) (layer B.Cu) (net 14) (status 10))
 (segment (start 157.734 78.74) (end 156.718 77.724) (width 0.25) (layer F.Cu) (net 14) (status 20))
 (segment (start 157.734 84.074) (end 157.734 78.74) (width 0.25) (layer F.Cu) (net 14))
 (via (at 157.734 84.074) (size 0.6) (drill 0.4) (layers F.Cu B.Cu) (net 14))
 (segment (start 157.734 88.9) (end 157.734 84.074) (width 0.25) (layer B.Cu) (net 14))
 (segment (start 156.718 77.724) (end 155.956 77.724) (width 0.25) (layer F.Cu) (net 14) (status 30))
 (segment (start 148.844 97.79) (end 149.86 97.79) (width 0.25) (layer F.Cu) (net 14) (status 30))
 (segment (start 149.86 97.79) (end 152.908 94.742) (width 0.25) (layer F.Cu) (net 14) (status 10))
 (via (at 152.908 94.742) (size 0.6) (drill 0.4) (layers F.Cu B.Cu) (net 14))
 (segment (start 152.908 94.742) (end 155.956 91.694) (width 0.25) (layer B.Cu) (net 14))
 (segment (start 155.956 91.694) (end 155.956 90.424) (width 0.25) (layer B.Cu) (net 14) (status 20))
 (segment (start 146.542 83.753) (end 146.542 86.064002) (width 0.25) (layer F.Cu) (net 20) (status 10))
 (segment (start 153.162 80.264) (end 155.956 80.264) (width 0.25) (layer B.Cu) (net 20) (status 20))
 (segment (start 152.654 80.772) (end 153.162 80.264) (width 0.25) (layer B.Cu) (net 20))
 (segment (start 152.654 82.296) (end 152.654 80.772) (width 0.25) (layer B.Cu) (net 20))
 (via (at 152.654 82.296) (size 0.6) (drill 0.4) (layers F.Cu B.Cu) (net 20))
 (segment (start 152.654 84.582) (end 152.654 82.296) (width 0.25) (layer F.Cu) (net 20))
 (segment (start 150.114 87.122) (end 152.654 84.582) (width 0.25) (layer F.Cu) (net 20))
 (segment (start 147.599998 87.122) (end 150.114 87.122) (width 0.25) (layer F.Cu) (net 20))
 (segment (start 146.542 86.064002) (end 147.599998 87.122) (width 0.25) (layer F.Cu) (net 20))
 (segment (start 147.507 81.288) (end 153.17 81.288) (width 0.25) (layer F.Cu) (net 21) (status 10))
 (segment (start 153.924 82.042) (end 154.686 82.804) (width 0.25) (layer B.Cu) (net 21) (status 20))
 (via (at 153.924 82.042) (size 0.6) (drill 0.4) (layers F.Cu B.Cu) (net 21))
 (segment (start 153.17 81.288) (end 153.924 82.042) (width 0.25) (layer F.Cu) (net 21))
 (segment (start 154.686 82.804) (end 155.956 82.804) (width 0.25) (layer B.Cu) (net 21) (status 30))
 (segment (start 152.642 87.884) (end 153.924 87.884) (width 0.25) (layer F.Cu) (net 22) (status 10))
 (segment (start 153.924 87.884) (end 155.956 87.884) (width 0.25) (layer B.Cu) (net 22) (status 20))
 (via (at 153.924 87.884) (size 0.6) (drill 0.4) (layers F.Cu B.Cu) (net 22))
 (segment (start 135.76808 79.89316) (end 135.76808 85.39226) (width 0.25) (layer F.Cu) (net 24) (status 30))
 (segment (start 126.86792 79.89316) (end 135.76808 79.89316) (width 0.25) (layer F.Cu) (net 24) (status 30))
 (segment (start 126.86792 85.39226) (end 126.86792 79.89316) (width 0.25) (layer F.Cu) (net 24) (status 30))
 (segment (start 127.242 89.154) (end 128.27 89.154) (width 0.25) (layer F.Cu) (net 25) (status 10))
 (segment (start 141.232 81.288) (end 143.577 81.288) (width 0.25) (layer F.Cu) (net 25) (status 20))
 (segment (start 141.224 81.28) (end 141.232 81.288) (width 0.25) (layer F.Cu) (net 25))
 (via (at 141.224 81.28) (size 0.6) (drill 0.4) (layers F.Cu B.Cu) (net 25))
 (segment (start 132.08 81.28) (end 141.224 81.28) (width 0.25) (layer B.Cu) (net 25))
 (segment (start 128.016 85.344) (end 132.08 81.28) (width 0.25) (layer B.Cu) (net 25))
 (segment (start 128.016 88.9) (end 128.016 85.344) (width 0.25) (layer B.Cu) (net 25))
 (segment (start 128.27 89.154) (end 128.016 88.9) (width 0.25) (layer B.Cu) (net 25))
 (via (at 128.27 89.154) (size 0.6) (drill 0.4) (layers F.Cu B.Cu) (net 25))
 (segment (start 143.577 80.788) (end 142.256 80.788) (width 0.25) (layer F.Cu) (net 26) (status 10))
 (segment (start 135.636 89.154) (end 134.862 89.154) (width 0.25) (layer F.Cu) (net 26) (status 20))
 (segment (start 137.414 87.376) (end 135.636 89.154) (width 0.25) (layer F.Cu) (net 26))
 (segment (start 137.414 80.772) (end 137.414 87.376) (width 0.25) (layer F.Cu) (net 26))
 (segment (start 137.668 80.518) (end 137.414 80.772) (width 0.25) (layer F.Cu) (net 26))
 (segment (start 141.986 80.518) (end 137.668 80.518) (width 0.25) (layer F.Cu) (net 26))
 (segment (start 142.256 80.788) (end 141.986 80.518) (width 0.25) (layer F.Cu) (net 26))
 (segment (start 143.764 97.04) (end 143.764 96.774) (width 0.25) (layer F.Cu) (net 27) (status 10))
 (segment (start 146.05 86.614) (end 146.05 84.074) (width 0.25) (layer F.Cu) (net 27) (status 20))
 (segment (start 146.304 86.868) (end 146.05 86.614) (width 0.25) (layer F.Cu) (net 27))
 (via (at 146.304 86.868) (size 0.6) (drill 0.4) (layers F.Cu B.Cu) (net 27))
 (segment (start 146.304 94.234) (end 146.304 86.868) (width 0.25) (layer B.Cu) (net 27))
 (segment (start 146.05 94.488) (end 146.304 94.234) (width 0.25) (layer B.Cu) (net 27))
 (via (at 146.05 94.488) (size 0.6) (drill 0.4) (layers F.Cu B.Cu) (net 27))
 (segment (start 143.764 96.774) (end 146.05 94.488) (width 0.25) (layer F.Cu) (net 27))
 (segment (start 146.05 84.074) (end 146.042 83.753) (width 0.25) (layer F.Cu) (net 27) (status 30))
 (segment (start 145.542 83.753) (end 145.542 87.884) (width 0.25) (layer F.Cu) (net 28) (status 10))
 (segment (start 145.542 87.884) (end 151.142 87.884) (width 0.25) (layer F.Cu) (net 28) (status 20)))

